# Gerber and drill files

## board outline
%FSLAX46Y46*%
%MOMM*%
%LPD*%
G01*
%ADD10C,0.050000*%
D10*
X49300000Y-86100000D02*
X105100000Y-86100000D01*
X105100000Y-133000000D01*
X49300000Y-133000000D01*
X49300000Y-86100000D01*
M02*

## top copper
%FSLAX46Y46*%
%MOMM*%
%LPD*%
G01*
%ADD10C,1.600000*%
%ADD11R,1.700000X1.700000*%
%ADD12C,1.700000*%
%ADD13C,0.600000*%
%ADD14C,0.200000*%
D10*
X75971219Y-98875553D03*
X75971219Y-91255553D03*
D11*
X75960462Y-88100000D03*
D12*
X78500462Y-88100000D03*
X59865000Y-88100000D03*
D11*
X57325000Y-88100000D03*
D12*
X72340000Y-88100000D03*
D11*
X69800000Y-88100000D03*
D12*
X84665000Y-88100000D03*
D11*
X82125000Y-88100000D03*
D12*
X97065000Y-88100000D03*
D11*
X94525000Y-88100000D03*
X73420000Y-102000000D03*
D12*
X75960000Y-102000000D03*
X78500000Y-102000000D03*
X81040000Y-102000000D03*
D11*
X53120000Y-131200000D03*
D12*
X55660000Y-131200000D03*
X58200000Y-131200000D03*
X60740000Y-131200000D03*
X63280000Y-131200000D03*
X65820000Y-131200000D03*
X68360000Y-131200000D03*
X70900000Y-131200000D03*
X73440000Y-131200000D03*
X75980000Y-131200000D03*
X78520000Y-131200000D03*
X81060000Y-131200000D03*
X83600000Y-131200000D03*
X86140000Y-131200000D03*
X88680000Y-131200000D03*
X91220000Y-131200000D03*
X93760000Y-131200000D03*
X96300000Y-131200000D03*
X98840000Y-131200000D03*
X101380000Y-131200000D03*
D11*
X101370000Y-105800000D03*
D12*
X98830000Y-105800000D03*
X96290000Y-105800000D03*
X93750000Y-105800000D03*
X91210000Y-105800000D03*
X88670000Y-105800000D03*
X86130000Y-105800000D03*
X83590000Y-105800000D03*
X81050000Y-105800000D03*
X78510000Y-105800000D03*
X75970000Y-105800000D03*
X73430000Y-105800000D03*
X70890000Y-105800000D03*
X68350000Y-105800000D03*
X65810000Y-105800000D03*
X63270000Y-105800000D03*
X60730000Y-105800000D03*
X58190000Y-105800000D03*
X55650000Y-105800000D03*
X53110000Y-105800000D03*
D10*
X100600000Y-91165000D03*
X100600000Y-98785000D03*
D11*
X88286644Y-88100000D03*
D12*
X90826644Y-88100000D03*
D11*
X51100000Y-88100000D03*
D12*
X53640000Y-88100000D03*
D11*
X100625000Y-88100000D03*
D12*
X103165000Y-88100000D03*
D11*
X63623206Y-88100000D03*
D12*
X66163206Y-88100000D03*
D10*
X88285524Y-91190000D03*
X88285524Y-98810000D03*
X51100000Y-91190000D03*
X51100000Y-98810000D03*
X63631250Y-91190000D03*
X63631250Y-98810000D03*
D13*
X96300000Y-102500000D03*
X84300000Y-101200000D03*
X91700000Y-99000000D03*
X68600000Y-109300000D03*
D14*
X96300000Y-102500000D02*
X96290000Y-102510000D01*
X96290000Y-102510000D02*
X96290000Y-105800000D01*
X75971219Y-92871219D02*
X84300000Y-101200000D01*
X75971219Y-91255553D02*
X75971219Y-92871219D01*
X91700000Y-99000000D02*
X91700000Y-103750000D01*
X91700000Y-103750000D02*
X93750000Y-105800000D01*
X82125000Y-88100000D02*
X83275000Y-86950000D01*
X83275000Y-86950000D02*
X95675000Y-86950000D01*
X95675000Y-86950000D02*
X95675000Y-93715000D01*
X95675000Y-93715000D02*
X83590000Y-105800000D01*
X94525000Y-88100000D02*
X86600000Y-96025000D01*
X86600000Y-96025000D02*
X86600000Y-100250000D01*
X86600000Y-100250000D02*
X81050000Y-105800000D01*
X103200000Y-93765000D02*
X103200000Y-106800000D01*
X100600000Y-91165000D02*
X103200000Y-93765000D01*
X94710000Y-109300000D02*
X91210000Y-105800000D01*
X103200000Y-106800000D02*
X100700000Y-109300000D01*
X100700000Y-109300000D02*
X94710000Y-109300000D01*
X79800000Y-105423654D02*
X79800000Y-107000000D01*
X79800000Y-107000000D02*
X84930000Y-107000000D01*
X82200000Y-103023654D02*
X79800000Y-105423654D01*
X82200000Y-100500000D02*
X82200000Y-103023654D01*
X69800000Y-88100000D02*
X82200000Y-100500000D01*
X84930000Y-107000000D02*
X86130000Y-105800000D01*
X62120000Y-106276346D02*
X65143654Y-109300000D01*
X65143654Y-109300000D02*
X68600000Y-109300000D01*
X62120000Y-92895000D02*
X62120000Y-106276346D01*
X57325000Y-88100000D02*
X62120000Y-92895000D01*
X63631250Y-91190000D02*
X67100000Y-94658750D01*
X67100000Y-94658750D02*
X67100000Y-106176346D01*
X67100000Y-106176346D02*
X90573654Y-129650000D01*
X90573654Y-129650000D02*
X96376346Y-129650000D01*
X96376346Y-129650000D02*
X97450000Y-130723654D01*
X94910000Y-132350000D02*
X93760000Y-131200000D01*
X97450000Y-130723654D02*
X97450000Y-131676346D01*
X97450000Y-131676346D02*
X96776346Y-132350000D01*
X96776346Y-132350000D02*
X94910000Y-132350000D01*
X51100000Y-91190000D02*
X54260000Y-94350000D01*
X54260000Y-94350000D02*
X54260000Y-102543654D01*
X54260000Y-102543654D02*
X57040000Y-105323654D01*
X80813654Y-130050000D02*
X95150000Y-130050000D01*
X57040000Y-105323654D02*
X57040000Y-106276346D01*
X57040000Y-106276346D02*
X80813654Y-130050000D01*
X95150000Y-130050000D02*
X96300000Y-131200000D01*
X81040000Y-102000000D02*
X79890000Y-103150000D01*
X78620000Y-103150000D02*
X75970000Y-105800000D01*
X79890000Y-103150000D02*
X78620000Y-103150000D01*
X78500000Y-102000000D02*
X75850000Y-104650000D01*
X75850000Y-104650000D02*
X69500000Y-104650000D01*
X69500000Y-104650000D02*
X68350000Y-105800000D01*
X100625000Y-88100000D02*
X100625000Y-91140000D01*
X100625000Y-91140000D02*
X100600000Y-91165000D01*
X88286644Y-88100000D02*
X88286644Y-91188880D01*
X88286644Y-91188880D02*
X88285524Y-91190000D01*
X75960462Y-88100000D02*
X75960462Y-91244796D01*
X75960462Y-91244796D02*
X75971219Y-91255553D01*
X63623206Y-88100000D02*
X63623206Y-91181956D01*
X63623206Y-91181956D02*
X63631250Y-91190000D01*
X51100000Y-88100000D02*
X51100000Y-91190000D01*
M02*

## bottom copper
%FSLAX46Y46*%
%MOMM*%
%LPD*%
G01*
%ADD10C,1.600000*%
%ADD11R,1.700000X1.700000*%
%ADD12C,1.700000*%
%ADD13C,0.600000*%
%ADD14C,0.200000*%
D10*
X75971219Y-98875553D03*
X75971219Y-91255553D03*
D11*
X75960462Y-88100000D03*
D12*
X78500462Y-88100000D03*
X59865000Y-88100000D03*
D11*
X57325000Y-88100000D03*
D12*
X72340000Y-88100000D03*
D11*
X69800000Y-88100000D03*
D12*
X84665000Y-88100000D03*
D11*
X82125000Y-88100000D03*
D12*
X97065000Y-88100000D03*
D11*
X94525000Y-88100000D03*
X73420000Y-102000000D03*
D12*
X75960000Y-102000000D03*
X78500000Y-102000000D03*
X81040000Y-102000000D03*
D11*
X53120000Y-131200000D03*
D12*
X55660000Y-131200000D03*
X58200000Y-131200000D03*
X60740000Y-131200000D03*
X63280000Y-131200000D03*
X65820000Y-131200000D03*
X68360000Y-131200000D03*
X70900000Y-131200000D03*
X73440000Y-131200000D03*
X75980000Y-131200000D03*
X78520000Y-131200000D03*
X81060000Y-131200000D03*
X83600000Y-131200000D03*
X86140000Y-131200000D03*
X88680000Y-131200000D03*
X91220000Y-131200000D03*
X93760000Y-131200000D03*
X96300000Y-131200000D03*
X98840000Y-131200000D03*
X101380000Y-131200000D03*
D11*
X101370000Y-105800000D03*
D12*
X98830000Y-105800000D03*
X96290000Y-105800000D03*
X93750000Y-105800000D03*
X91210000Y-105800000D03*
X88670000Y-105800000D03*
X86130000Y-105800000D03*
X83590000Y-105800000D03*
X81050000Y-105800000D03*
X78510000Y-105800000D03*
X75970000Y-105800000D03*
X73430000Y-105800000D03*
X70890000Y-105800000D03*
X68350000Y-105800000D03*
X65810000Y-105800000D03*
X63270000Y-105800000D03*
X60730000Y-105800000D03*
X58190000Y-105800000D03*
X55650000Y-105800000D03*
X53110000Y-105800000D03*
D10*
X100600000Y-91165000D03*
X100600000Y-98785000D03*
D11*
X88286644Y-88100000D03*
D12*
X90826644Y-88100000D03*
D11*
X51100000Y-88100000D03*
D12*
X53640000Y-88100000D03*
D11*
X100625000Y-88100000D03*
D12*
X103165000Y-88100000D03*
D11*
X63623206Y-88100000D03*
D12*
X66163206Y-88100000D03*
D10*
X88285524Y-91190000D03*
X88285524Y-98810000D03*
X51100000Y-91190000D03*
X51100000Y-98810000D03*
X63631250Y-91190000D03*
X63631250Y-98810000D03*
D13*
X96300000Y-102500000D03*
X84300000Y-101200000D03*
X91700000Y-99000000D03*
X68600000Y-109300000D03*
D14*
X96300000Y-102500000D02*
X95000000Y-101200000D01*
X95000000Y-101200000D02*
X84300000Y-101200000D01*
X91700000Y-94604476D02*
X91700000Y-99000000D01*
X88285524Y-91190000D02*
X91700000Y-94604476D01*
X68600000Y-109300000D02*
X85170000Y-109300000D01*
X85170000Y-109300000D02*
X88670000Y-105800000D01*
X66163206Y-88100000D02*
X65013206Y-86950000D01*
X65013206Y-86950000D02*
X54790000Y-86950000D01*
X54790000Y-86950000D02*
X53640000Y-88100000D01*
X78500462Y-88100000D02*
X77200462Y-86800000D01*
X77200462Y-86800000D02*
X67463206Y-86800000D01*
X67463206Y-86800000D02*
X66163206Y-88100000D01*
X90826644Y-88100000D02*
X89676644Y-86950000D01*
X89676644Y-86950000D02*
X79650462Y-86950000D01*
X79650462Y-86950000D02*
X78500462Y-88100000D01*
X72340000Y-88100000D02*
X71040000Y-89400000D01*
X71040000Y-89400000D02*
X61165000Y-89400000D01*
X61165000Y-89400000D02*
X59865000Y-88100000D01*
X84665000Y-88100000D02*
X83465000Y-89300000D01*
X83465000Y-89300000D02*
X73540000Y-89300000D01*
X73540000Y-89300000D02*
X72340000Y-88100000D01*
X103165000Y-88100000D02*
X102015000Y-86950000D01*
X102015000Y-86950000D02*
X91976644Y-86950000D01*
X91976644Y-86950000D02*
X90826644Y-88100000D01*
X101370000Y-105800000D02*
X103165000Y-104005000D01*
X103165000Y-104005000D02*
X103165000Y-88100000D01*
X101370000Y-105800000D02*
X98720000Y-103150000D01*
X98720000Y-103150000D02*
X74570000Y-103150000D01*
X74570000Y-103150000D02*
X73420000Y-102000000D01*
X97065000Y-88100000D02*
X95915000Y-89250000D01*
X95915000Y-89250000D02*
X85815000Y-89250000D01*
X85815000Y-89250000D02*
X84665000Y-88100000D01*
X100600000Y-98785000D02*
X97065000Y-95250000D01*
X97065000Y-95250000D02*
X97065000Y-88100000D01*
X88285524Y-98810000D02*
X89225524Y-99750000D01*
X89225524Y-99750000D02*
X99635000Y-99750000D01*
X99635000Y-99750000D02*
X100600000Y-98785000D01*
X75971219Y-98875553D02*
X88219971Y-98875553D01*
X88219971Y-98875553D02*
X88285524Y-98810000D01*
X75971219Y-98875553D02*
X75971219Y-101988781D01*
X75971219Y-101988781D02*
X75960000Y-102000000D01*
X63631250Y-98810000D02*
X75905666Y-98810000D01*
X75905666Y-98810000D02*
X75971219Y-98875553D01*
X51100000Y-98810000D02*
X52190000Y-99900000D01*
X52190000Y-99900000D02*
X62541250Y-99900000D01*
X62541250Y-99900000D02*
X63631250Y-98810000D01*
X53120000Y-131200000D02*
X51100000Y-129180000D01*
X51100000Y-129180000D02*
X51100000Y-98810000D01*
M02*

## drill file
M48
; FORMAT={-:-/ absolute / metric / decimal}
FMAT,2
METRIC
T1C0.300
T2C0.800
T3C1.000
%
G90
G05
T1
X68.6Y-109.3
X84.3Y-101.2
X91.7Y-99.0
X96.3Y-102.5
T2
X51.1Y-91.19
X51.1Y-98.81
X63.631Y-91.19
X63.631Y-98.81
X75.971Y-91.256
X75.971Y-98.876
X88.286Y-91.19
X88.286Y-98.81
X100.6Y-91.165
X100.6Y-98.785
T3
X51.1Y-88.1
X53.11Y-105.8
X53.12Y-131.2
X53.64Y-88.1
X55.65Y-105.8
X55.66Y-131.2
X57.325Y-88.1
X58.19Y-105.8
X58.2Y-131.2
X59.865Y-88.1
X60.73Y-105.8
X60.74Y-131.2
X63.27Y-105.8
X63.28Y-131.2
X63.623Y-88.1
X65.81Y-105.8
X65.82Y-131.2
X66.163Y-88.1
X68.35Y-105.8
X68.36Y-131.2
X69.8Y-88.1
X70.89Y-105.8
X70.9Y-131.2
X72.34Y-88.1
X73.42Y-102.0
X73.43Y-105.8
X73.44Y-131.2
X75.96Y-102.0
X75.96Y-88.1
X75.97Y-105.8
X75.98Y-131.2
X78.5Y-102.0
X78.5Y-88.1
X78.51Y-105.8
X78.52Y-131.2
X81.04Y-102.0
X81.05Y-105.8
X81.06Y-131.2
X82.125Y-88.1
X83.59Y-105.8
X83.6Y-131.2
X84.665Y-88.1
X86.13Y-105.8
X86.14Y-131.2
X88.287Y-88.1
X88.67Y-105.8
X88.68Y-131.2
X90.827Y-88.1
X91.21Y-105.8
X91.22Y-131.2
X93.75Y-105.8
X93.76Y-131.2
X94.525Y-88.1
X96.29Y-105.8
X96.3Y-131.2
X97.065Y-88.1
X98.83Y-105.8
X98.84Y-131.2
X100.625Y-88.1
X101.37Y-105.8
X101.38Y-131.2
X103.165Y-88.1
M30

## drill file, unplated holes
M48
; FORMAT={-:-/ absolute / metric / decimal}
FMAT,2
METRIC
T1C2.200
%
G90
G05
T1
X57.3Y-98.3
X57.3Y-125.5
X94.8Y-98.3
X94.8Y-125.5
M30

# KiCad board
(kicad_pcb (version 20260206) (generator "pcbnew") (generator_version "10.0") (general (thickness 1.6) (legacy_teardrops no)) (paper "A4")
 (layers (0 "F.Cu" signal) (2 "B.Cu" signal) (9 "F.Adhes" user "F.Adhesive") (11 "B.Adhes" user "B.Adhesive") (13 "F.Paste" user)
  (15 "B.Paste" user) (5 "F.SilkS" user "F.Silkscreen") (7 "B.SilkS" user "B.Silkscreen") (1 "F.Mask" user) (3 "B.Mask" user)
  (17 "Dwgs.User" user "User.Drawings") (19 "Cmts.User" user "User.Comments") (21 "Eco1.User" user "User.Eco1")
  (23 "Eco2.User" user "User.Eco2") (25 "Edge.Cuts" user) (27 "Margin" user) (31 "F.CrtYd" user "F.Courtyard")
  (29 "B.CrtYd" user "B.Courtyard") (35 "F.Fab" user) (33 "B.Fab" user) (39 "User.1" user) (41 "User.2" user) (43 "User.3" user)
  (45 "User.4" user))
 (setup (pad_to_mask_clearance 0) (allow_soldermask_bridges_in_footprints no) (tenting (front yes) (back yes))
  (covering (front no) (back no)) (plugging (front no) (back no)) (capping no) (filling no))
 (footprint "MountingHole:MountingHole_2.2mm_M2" (layer "F.Cu") (at 94.8 125.5)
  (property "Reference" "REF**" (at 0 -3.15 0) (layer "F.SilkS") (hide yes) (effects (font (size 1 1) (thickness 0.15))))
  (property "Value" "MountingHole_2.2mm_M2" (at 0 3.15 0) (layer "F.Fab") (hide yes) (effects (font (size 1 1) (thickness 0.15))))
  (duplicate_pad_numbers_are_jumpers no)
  (pad "" np_thru_hole circle (at 0 0) (size 2.2 2.2) (drill 2.2) (layers "*.Cu" "*.Mask")))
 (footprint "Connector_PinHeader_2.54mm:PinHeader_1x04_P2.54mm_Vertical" (layer "F.Cu") (at 73.42 102 90)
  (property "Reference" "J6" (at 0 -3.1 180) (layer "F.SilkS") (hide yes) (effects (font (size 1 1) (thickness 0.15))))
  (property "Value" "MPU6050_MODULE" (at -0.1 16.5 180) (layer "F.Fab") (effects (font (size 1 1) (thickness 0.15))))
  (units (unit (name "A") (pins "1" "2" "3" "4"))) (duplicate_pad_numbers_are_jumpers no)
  (pad "1" thru_hole rect (at 0 0 90) (size 1.7 1.7) (drill 1) (layers "*.Cu" "*.Mask") (remove_unused_layers no) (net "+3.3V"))
  (pad "2" thru_hole circle (at 0 2.54 90) (size 1.7 1.7) (drill 1) (layers "*.Cu" "*.Mask") (remove_unused_layers no) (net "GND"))
  (pad "3" thru_hole circle (at 0 5.08 90) (size 1.7 1.7) (drill 1) (layers "*.Cu" "*.Mask") (remove_unused_layers no) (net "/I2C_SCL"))
  (pad "4" thru_hole circle (at 0 7.62 90) (size 1.7 1.7) (drill 1) (layers "*.Cu" "*.Mask") (remove_unused_layers no) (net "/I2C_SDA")))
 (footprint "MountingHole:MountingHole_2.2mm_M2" (layer "F.Cu") (at 94.8 98.3)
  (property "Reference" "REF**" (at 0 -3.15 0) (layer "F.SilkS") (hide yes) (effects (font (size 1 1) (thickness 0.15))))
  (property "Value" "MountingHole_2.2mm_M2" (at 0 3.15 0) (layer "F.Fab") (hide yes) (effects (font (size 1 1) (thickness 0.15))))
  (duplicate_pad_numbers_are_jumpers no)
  (pad "" np_thru_hole circle (at 0 0) (size 2.2 2.2) (drill 2.2) (layers "*.Cu" "*.Mask")))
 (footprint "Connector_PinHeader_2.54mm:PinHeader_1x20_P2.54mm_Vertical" (layer "F.Cu") (at 53.12 131.2 90)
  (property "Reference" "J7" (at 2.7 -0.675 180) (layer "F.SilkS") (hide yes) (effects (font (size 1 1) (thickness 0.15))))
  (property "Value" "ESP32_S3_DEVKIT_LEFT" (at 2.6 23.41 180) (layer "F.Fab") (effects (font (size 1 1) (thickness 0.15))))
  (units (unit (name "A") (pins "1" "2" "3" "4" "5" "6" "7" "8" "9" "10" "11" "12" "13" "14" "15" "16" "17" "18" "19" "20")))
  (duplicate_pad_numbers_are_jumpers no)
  (pad "1" thru_hole rect (at 0 0 90) (size 1.7 1.7) (drill 1) (layers "*.Cu" "*.Mask") (remove_unused_layers no) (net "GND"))
  (pad "2" thru_hole circle (at 0 2.54 90) (size 1.7 1.7) (drill 1) (layers "*.Cu" "*.Mask") (remove_unused_layers no)
   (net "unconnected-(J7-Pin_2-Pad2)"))
  (pad "3" thru_hole circle (at 0 5.08 90) (size 1.7 1.7) (drill 1) (layers "*.Cu" "*.Mask") (remove_unused_layers no)
   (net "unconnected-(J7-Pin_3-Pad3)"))
  (pad "4" thru_hole circle (at 0 7.62 90) (size 1.7 1.7) (drill 1) (layers "*.Cu" "*.Mask") (remove_unused_layers no)
   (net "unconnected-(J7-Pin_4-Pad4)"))
  (pad "5" thru_hole circle (at 0 10.16 90) (size 1.7 1.7) (drill 1) (layers "*.Cu" "*.Mask") (remove_unused_layers no)
   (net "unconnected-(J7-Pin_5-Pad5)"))
  (pad "6" thru_hole circle (at 0 12.7 90) (size 1.7 1.7) (drill 1) (layers "*.Cu" "*.Mask") (remove_unused_layers no)
   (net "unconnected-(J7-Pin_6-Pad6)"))
  (pad "7" thru_hole circle (at 0 15.24 90) (size 1.7 1.7) (drill 1) (layers "*.Cu" "*.Mask") (remove_unused_layers no)
   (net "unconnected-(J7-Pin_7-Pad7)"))
  (pad "8" thru_hole circle (at 0 17.78 90) (size 1.7 1.7) (drill 1) (layers "*.Cu" "*.Mask") (remove_unused_layers no)
   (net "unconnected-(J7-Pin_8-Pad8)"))
  (pad "9" thru_hole circle (at 0 20.32 90) (size 1.7 1.7) (drill 1) (layers "*.Cu" "*.Mask") (remove_unused_layers no)
   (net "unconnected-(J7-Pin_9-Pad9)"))
  (pad "10" thru_hole circle (at 0 22.86 90) (size 1.7 1.7) (drill 1) (layers "*.Cu" "*.Mask") (remove_unused_layers no)
   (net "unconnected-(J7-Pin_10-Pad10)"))
  (pad "11" thru_hole circle (at 0 25.4 90) (size 1.7 1.7) (drill 1) (layers "*.Cu" "*.Mask") (remove_unused_layers no)
   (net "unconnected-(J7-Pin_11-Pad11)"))
  (pad "12" thru_hole circle (at 0 27.94 90) (size 1.7 1.7) (drill 1) (layers "*.Cu" "*.Mask") (remove_unused_layers no)
   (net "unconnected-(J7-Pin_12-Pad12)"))
  (pad "13" thru_hole circle (at 0 30.48 90) (size 1.7 1.7) (drill 1) (layers "*.Cu" "*.Mask") (remove_unused_layers no)
   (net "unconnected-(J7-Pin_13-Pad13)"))
  (pad "14" thru_hole circle (at 0 33.02 90) (size 1.7 1.7) (drill 1) (layers "*.Cu" "*.Mask") (remove_unused_layers no)
   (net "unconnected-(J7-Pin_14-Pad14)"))
  (pad "15" thru_hole circle (at 0 35.56 90) (size 1.7 1.7) (drill 1) (layers "*.Cu" "*.Mask") (remove_unused_layers no)
   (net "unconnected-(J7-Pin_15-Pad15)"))
  (pad "16" thru_hole circle (at 0 38.1 90) (size 1.7 1.7) (drill 1) (layers "*.Cu" "*.Mask") (remove_unused_layers no)
   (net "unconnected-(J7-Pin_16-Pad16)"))
  (pad "17" thru_hole circle (at 0 40.64 90) (size 1.7 1.7) (drill 1) (layers "*.Cu" "*.Mask") (remove_unused_layers no) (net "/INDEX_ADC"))
  (pad "18" thru_hole circle (at 0 43.18 90) (size 1.7 1.7) (drill 1) (layers "*.Cu" "*.Mask") (remove_unused_layers no) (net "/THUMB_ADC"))
  (pad "19" thru_hole circle (at 0 45.72 90) (size 1.7 1.7) (drill 1) (layers "*.Cu" "*.Mask") (remove_unused_layers no)
   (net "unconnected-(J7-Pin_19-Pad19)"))
  (pad "20" thru_hole circle (at 0 48.26 90) (size 1.7 1.7) (drill 1) (layers "*.Cu" "*.Mask") (remove_unused_layers no)
   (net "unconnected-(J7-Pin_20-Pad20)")))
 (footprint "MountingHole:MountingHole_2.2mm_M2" (layer "F.Cu") (at 57.3 98.3)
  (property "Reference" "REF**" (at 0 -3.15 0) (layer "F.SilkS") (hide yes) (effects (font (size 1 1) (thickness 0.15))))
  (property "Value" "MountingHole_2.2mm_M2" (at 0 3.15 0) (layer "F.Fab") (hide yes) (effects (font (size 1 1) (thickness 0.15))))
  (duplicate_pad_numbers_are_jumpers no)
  (pad "" np_thru_hole circle (at 0 0) (size 2.2 2.2) (drill 2.2) (layers "*.Cu" "*.Mask")))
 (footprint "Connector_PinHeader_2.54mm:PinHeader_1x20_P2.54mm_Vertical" (layer "F.Cu") (at 101.37 105.8 -90)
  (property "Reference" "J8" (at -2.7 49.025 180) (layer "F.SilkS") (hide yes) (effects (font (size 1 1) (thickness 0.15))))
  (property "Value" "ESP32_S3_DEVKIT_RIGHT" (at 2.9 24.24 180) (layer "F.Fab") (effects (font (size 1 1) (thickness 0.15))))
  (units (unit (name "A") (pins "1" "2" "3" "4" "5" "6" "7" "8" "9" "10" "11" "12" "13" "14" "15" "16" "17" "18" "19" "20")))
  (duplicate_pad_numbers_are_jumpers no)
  (pad "1" thru_hole rect (at 0 0 270) (size 1.7 1.7) (drill 1) (layers "*.Cu" "*.Mask") (remove_unused_layers no) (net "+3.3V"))
  (pad "2" thru_hole circle (at 0 2.54 270) (size 1.7 1.7) (drill 1) (layers "*.Cu" "*.Mask") (remove_unused_layers no)
   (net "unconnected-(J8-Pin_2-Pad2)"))
  (pad "3" thru_hole circle (at 0 5.08 270) (size 1.7 1.7) (drill 1) (layers "*.Cu" "*.Mask") (remove_unused_layers no) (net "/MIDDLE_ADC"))
  (pad "4" thru_hole circle (at 0 7.62 270) (size 1.7 1.7) (drill 1) (layers "*.Cu" "*.Mask") (remove_unused_layers no) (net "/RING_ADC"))
  (pad "5" thru_hole circle (at 0 10.16 270) (size 1.7 1.7) (drill 1) (layers "*.Cu" "*.Mask") (remove_unused_layers no) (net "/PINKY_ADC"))
  (pad "6" thru_hole circle (at 0 12.7 270) (size 1.7 1.7) (drill 1) (layers "*.Cu" "*.Mask") (remove_unused_layers no) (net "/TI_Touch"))
  (pad "7" thru_hole circle (at 0 15.24 270) (size 1.7 1.7) (drill 1) (layers "*.Cu" "*.Mask") (remove_unused_layers no) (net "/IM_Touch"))
  (pad "8" thru_hole circle (at 0 17.78 270) (size 1.7 1.7) (drill 1) (layers "*.Cu" "*.Mask") (remove_unused_layers no) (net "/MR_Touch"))
  (pad "9" thru_hole circle (at 0 20.32 270) (size 1.7 1.7) (drill 1) (layers "*.Cu" "*.Mask") (remove_unused_layers no) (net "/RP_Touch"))
  (pad "10" thru_hole circle (at 0 22.86 270) (size 1.7 1.7) (drill 1) (layers "*.Cu" "*.Mask") (remove_unused_layers no)
   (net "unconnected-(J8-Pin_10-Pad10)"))
  (pad "11" thru_hole circle (at 0 25.4 270) (size 1.7 1.7) (drill 1) (layers "*.Cu" "*.Mask") (remove_unused_layers no) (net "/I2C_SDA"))
  (pad "12" thru_hole circle (at 0 27.94 270) (size 1.7 1.7) (drill 1) (layers "*.Cu" "*.Mask") (remove_unused_layers no)
   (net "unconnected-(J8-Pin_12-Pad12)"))
  (pad "13" thru_hole circle (at 0 30.48 270) (size 1.7 1.7) (drill 1) (layers "*.Cu" "*.Mask") (remove_unused_layers no)
   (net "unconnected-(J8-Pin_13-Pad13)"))
  (pad "14" thru_hole circle (at 0 33.02 270) (size 1.7 1.7) (drill 1) (layers "*.Cu" "*.Mask") (remove_unused_layers no) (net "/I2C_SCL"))
  (pad "15" thru_hole circle (at 0 35.56 270) (size 1.7 1.7) (drill 1) (layers "*.Cu" "*.Mask") (remove_unused_layers no)
   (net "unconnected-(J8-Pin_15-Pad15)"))
  (pad "16" thru_hole circle (at 0 38.1 270) (size 1.7 1.7) (drill 1) (layers "*.Cu" "*.Mask") (remove_unused_layers no)
   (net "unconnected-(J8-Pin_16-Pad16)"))
  (pad "17" thru_hole circle (at 0 40.64 270) (size 1.7 1.7) (drill 1) (layers "*.Cu" "*.Mask") (remove_unused_layers no)
   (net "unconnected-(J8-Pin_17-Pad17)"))
  (pad "18" thru_hole circle (at 0 43.18 270) (size 1.7 1.7) (drill 1) (layers "*.Cu" "*.Mask") (remove_unused_layers no)
   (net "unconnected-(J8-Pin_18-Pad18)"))
  (pad "19" thru_hole circle (at 0 45.72 270) (size 1.7 1.7) (drill 1) (layers "*.Cu" "*.Mask") (remove_unused_layers no)
   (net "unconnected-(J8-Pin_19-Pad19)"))
  (pad "20" thru_hole circle (at 0 48.26 270) (size 1.7 1.7) (drill 1) (layers "*.Cu" "*.Mask") (remove_unused_layers no)
   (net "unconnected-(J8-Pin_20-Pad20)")))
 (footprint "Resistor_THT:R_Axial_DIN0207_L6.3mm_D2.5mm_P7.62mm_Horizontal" (layer "F.Cu") (at 100.6 91.165 -90)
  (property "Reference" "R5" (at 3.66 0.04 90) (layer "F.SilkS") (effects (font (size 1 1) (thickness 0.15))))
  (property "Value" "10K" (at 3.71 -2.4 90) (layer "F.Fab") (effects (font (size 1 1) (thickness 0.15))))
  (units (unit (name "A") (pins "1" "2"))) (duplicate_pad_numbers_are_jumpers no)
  (pad "1" thru_hole circle (at 0 0 270) (size 1.6 1.6) (drill 0.8) (layers "*.Cu" "*.Mask") (remove_unused_layers no) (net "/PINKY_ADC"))
  (pad "2" thru_hole circle (at 7.62 0 270) (size 1.6 1.6) (drill 0.8) (layers "*.Cu" "*.Mask") (remove_unused_layers no) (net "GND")))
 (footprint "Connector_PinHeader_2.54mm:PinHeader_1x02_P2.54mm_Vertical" (layer "F.Cu") (at 82.125 88.1 90)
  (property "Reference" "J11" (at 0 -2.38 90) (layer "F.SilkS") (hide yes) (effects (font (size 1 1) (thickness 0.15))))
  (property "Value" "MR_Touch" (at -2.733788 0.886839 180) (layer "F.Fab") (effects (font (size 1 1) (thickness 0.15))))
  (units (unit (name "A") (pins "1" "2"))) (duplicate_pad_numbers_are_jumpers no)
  (pad "1" thru_hole rect (at 0 0 90) (size 1.7 1.7) (drill 1) (layers "*.Cu" "*.Mask") (remove_unused_layers no) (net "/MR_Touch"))
  (pad "2" thru_hole circle (at 0 2.54 90) (size 1.7 1.7) (drill 1) (layers "*.Cu" "*.Mask") (remove_unused_layers no) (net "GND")))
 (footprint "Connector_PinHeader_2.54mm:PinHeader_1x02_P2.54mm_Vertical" (layer "F.Cu") (at 94.525 88.1 90)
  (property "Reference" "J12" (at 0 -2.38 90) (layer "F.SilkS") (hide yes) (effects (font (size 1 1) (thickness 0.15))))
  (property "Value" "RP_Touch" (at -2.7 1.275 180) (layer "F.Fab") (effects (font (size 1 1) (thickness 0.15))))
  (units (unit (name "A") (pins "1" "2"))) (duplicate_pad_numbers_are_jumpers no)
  (pad "1" thru_hole rect (at 0 0 90) (size 1.7 1.7) (drill 1) (layers "*.Cu" "*.Mask") (remove_unused_layers no) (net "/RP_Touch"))
  (pad "2" thru_hole circle (at 0 2.54 90) (size 1.7 1.7) (drill 1) (layers "*.Cu" "*.Mask") (remove_unused_layers no) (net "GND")))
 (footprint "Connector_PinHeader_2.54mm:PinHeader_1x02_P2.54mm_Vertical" (layer "F.Cu") (at 88.286644 88.1 90)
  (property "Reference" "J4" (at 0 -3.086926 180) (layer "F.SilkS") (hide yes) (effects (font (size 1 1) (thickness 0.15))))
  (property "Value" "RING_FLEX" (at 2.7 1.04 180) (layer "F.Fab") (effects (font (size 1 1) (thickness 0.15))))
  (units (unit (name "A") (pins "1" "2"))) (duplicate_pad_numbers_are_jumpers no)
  (pad "1" thru_hole rect (at 0 0 90) (size 1.7 1.7) (drill 1) (layers "*.Cu" "*.Mask") (remove_unused_layers no) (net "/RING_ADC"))
  (pad "2" thru_hole circle (at 0 2.54 90) (size 1.7 1.7) (drill 1) (layers "*.Cu" "*.Mask") (remove_unused_layers no) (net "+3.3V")))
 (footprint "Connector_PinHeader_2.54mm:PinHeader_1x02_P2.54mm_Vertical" (layer "F.Cu") (at 51.1 88.1 90)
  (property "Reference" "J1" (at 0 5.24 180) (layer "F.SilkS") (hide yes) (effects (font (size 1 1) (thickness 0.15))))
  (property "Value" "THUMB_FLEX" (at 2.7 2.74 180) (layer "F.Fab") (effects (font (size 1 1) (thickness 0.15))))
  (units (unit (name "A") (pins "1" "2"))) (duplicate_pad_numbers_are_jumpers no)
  (pad "1" thru_hole rect (at 0 0 90) (size 1.7 1.7) (drill 1) (layers "*.Cu" "*.Mask") (remove_unused_layers no) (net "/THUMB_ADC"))
  (pad "2" thru_hole circle (at 0 2.54 90) (size 1.7 1.7) (drill 1) (layers "*.Cu" "*.Mask") (remove_unused_layers no) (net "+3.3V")))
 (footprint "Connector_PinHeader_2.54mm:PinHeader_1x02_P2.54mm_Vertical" (layer "F.Cu") (at 100.625 88.1 90)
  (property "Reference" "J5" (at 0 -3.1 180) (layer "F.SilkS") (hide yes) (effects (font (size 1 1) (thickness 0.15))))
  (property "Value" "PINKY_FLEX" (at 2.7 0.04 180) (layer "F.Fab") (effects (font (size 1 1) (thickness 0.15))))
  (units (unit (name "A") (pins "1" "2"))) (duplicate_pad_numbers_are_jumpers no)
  (pad "1" thru_hole rect (at 0 0 90) (size 1.7 1.7) (drill 1) (layers "*.Cu" "*.Mask") (remove_unused_layers no) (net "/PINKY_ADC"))
  (pad "2" thru_hole circle (at 0 2.54 90) (size 1.7 1.7) (drill 1) (layers "*.Cu" "*.Mask") (remove_unused_layers no) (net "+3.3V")))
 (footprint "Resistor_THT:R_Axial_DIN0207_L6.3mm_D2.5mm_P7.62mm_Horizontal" (layer "F.Cu") (at 75.971219 91.255553 -90)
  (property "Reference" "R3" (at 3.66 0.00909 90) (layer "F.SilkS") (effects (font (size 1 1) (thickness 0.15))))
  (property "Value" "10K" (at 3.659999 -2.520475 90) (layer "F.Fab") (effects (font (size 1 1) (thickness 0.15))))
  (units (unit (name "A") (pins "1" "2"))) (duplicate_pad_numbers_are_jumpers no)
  (pad "1" thru_hole circle (at 0 0 270) (size 1.6 1.6) (drill 0.8) (layers "*.Cu" "*.Mask") (remove_unused_layers no) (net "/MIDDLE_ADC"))
  (pad "2" thru_hole circle (at 7.62 0 270) (size 1.6 1.6) (drill 0.8) (layers "*.Cu" "*.Mask") (remove_unused_layers no) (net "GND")))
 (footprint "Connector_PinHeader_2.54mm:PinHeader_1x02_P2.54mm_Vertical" (layer "F.Cu") (at 63.623206 88.1 90)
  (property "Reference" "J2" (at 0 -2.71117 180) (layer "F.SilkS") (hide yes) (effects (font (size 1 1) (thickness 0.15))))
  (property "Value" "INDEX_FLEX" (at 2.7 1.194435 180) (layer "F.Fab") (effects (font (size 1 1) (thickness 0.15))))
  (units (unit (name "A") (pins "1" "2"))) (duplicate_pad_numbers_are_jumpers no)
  (pad "1" thru_hole rect (at 0 0 90) (size 1.7 1.7) (drill 1) (layers "*.Cu" "*.Mask") (remove_unused_layers no) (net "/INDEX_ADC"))
  (pad "2" thru_hole circle (at 0 2.54 90) (size 1.7 1.7) (drill 1) (layers "*.Cu" "*.Mask") (remove_unused_layers no) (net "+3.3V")))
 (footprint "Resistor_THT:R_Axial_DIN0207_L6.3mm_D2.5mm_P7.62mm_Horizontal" (layer "F.Cu") (at 88.285524 91.19 -90)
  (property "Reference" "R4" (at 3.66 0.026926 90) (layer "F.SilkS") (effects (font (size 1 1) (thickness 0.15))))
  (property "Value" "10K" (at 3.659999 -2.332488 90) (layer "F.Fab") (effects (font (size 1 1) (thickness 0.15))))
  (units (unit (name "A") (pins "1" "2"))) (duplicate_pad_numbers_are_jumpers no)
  (pad "1" thru_hole circle (at 0 0 270) (size 1.6 1.6) (drill 0.8) (layers "*.Cu" "*.Mask") (remove_unused_layers no) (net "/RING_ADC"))
  (pad "2" thru_hole circle (at 7.62 0 270) (size 1.6 1.6) (drill 0.8) (layers "*.Cu" "*.Mask") (remove_unused_layers no) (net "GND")))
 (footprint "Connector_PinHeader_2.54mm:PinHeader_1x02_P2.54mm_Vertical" (layer "F.Cu") (at 57.325 88.1 90)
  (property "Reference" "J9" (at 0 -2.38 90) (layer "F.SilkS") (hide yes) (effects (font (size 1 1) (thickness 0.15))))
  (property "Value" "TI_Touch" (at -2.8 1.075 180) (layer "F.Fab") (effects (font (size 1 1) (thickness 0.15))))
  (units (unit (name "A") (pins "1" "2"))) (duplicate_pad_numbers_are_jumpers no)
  (pad "1" thru_hole rect (at 0 0 90) (size 1.7 1.7) (drill 1) (layers "*.Cu" "*.Mask") (remove_unused_layers no) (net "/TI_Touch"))
  (pad "2" thru_hole circle (at 0 2.54 90) (size 1.7 1.7) (drill 1) (layers "*.Cu" "*.Mask") (remove_unused_layers no) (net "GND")))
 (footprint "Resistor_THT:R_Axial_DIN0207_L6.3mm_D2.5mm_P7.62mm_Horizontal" (layer "F.Cu") (at 51.1 91.19 -90)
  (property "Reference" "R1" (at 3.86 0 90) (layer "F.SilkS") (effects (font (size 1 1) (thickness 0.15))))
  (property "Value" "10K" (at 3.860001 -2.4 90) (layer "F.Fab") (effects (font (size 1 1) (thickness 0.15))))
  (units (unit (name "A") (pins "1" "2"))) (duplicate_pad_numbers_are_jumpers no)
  (pad "1" thru_hole circle (at 0 0 270) (size 1.6 1.6) (drill 0.8) (layers "*.Cu" "*.Mask") (remove_unused_layers no) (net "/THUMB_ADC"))
  (pad "2" thru_hole circle (at 7.62 0 270) (size 1.6 1.6) (drill 0.8) (layers "*.Cu" "*.Mask") (remove_unused_layers no) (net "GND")))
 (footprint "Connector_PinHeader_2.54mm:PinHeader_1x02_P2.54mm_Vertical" (layer "F.Cu") (at 75.960462 88.1 90)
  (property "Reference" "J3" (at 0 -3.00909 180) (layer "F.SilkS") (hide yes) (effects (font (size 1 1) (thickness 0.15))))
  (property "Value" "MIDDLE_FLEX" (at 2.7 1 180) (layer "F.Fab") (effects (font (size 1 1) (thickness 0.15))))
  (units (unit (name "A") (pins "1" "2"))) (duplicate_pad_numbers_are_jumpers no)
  (pad "1" thru_hole rect (at 0 0 90) (size 1.7 1.7) (drill 1) (layers "*.Cu" "*.Mask") (remove_unused_layers no) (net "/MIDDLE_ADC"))
  (pad "2" thru_hole circle (at 0 2.54 90) (size 1.7 1.7) (drill 1) (layers "*.Cu" "*.Mask") (remove_unused_layers no) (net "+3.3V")))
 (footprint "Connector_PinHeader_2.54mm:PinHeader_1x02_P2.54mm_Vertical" (layer "F.Cu") (at 69.8 88.1 90)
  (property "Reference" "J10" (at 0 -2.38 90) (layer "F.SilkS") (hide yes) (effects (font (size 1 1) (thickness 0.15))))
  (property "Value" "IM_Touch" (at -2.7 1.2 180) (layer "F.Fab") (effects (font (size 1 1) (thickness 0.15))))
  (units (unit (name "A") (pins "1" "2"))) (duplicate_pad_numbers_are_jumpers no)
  (pad "1" thru_hole rect (at 0 0 90) (size 1.7 1.7) (drill 1) (layers "*.Cu" "*.Mask") (remove_unused_layers no) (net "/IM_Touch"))
  (pad "2" thru_hole circle (at 0 2.54 90) (size 1.7 1.7) (drill 1) (layers "*.Cu" "*.Mask") (remove_unused_layers no) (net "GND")))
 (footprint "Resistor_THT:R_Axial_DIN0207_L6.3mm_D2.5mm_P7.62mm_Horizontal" (layer "F.Cu") (at 63.63125 91.19 -90)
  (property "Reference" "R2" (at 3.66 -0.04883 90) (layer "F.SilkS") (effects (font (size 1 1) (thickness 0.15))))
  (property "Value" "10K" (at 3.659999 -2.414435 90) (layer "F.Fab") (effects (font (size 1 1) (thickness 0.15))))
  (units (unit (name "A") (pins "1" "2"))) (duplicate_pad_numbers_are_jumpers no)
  (pad "1" thru_hole circle (at 0 0 270) (size 1.6 1.6) (drill 0.8) (layers "*.Cu" "*.Mask") (remove_unused_layers no) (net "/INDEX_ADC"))
  (pad "2" thru_hole circle (at 7.62 0 270) (size 1.6 1.6) (drill 0.8) (layers "*.Cu" "*.Mask") (remove_unused_layers no) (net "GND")))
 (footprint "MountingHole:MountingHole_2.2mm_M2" (layer "F.Cu") (at 57.3 125.5)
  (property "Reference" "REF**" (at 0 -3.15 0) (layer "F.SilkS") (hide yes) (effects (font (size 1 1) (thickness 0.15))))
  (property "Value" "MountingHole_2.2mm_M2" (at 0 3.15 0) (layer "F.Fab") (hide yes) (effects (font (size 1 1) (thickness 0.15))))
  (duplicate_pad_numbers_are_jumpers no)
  (pad "" np_thru_hole circle (at 0 0) (size 2.2 2.2) (drill 2.2) (layers "*.Cu" "*.Mask")))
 (gr_rect (start 49.3 86.1) (end 105.1 133) (stroke (width 0.05) (type default)) (fill no) (layer "Edge.Cuts"))
 (segment (start 77.200462 86.8) (end 67.463206 86.8) (width 0.2) (layer "B.Cu") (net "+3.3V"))
 (segment (start 79.650462 86.95) (end 78.500462 88.1) (width 0.2) (layer "B.Cu") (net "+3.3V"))
 (segment (start 98.72 103.15) (end 74.57 103.15) (width 0.2) (layer "B.Cu") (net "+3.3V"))
 (segment (start 103.165 88.1) (end 102.015 86.95) (width 0.2) (layer "B.Cu") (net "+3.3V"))
 (segment (start 91.976644 86.95) (end 90.826644 88.1) (width 0.2) (layer "B.Cu") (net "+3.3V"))
 (segment (start 90.826644 88.1) (end 89.676644 86.95) (width 0.2) (layer "B.Cu") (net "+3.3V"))
 (segment (start 89.676644 86.95) (end 79.650462 86.95) (width 0.2) (layer "B.Cu") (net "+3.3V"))
 (segment (start 65.013206 86.95) (end 54.79 86.95) (width 0.2) (layer "B.Cu") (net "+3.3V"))
 (segment (start 74.57 103.15) (end 73.42 102) (width 0.2) (layer "B.Cu") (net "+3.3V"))
 (segment (start 103.165 104.005) (end 103.165 88.1) (width 0.2) (layer "B.Cu") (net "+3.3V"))
 (segment (start 102.015 86.95) (end 91.976644 86.95) (width 0.2) (layer "B.Cu") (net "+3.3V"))
 (segment (start 78.500462 88.1) (end 77.200462 86.8) (width 0.2) (layer "B.Cu") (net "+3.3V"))
 (segment (start 67.463206 86.8) (end 66.163206 88.1) (width 0.2) (layer "B.Cu") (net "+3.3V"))
 (segment (start 101.37 105.8) (end 103.165 104.005) (width 0.2) (layer "B.Cu") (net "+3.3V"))
 (segment (start 66.163206 88.1) (end 65.013206 86.95) (width 0.2) (layer "B.Cu") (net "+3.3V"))
 (segment (start 54.79 86.95) (end 53.64 88.1) (width 0.2) (layer "B.Cu") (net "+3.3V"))
 (segment (start 101.37 105.8) (end 98.72 103.15) (width 0.2) (layer "B.Cu") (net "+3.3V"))
 (segment (start 51.1 98.81) (end 52.19 99.9) (width 0.2) (layer "B.Cu") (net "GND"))
 (segment (start 52.19 99.9) (end 62.54125 99.9) (width 0.2) (layer "B.Cu") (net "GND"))
 (segment (start 88.219971 98.875553) (end 88.285524 98.81) (width 0.2) (layer "B.Cu") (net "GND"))
 (segment (start 100.6 98.785) (end 97.065 95.25) (width 0.2) (layer "B.Cu") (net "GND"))
 (segment (start 85.815 89.25) (end 84.665 88.1) (width 0.2) (layer "B.Cu") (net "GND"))
 (segment (start 75.971219 98.875553) (end 88.219971 98.875553) (width 0.2) (layer "B.Cu") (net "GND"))
 (segment (start 63.63125 98.81) (end 75.905666 98.81) (width 0.2) (layer "B.Cu") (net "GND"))
 (segment (start 88.285524 98.81) (end 89.225524 99.75) (width 0.2) (layer "B.Cu") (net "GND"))
 (segment (start 51.1 129.18) (end 51.1 98.81) (width 0.2) (layer "B.Cu") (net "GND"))
 (segment (start 75.971219 101.988781) (end 75.96 102) (width 0.2) (layer "B.Cu") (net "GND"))
 (segment (start 62.54125 99.9) (end 63.63125 98.81) (width 0.2) (layer "B.Cu") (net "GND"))
 (segment (start 53.12 131.2) (end 51.1 129.18) (width 0.2) (layer "B.Cu") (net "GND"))
 (segment (start 89.225524 99.75) (end 99.635 99.75) (width 0.2) (layer "B.Cu") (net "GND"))
 (segment (start 97.065 95.25) (end 97.065 88.1) (width 0.2) (layer "B.Cu") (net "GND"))
 (segment (start 72.34 88.1) (end 71.04 89.4) (width 0.2) (layer "B.Cu") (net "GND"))
 (segment (start 97.065 88.1) (end 95.915 89.25) (width 0.2) (layer "B.Cu") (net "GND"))
 (segment (start 61.165 89.4) (end 59.865 88.1) (width 0.2) (layer "B.Cu") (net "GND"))
 (segment (start 75.971219 98.875553) (end 75.971219 101.988781) (width 0.2) (layer "B.Cu") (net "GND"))
 (segment (start 71.04 89.4) (end 61.165 89.4) (width 0.2) (layer "B.Cu") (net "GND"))
 (segment (start 75.905666 98.81) (end 75.971219 98.875553) (width 0.2) (layer "B.Cu") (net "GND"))
 (segment (start 99.635 99.75) (end 100.6 98.785) (width 0.2) (layer "B.Cu") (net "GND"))
 (segment (start 73.54 89.3) (end 72.34 88.1) (width 0.2) (layer "B.Cu") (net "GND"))
 (segment (start 84.665 88.1) (end 83.465 89.3) (width 0.2) (layer "B.Cu") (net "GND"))
 (segment (start 83.465 89.3) (end 73.54 89.3) (width 0.2) (layer "B.Cu") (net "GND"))
 (segment (start 95.915 89.25) (end 85.815 89.25) (width 0.2) (layer "B.Cu") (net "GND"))
 (segment (start 78.5 102) (end 75.85 104.65) (width 0.2) (layer "F.Cu") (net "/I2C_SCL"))
 (segment (start 69.5 104.65) (end 68.35 105.8) (width 0.2) (layer "F.Cu") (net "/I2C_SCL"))
 (segment (start 75.85 104.65) (end 69.5 104.65) (width 0.2) (layer "F.Cu") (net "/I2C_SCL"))
 (segment (start 78.62 103.15) (end 75.97 105.8) (width 0.2) (layer "F.Cu") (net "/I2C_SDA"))
 (segment (start 81.04 102) (end 79.89 103.15) (width 0.2) (layer "F.Cu") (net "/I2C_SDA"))
 (segment (start 79.89 103.15) (end 78.62 103.15) (width 0.2) (layer "F.Cu") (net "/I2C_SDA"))
 (segment (start 63.623206 91.181956) (end 63.63125 91.19) (width 0.2) (layer "F.Cu") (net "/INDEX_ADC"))
 (segment (start 63.63125 91.19) (end 67.1 94.65875) (width 0.2) (layer "F.Cu") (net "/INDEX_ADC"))
 (segment (start 67.1 106.176346) (end 90.573654 129.65) (width 0.2) (layer "F.Cu") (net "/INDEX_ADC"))
 (segment (start 97.45 130.723654) (end 97.45 131.676346) (width 0.2) (layer "F.Cu") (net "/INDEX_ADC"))
 (segment (start 96.376346 129.65) (end 97.45 130.723654) (width 0.2) (layer "F.Cu") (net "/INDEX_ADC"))
 (segment (start 96.776346 132.35) (end 94.91 132.35) (width 0.2) (layer "F.Cu") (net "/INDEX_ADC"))
 (segment (start 97.45 131.676346) (end 96.776346 132.35) (width 0.2) (layer "F.Cu") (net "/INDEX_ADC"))
 (segment (start 94.91 132.35) (end 93.76 131.2) (width 0.2) (layer "F.Cu") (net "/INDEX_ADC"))
 (segment (start 67.1 94.65875) (end 67.1 106.176346) (width 0.2) (layer "F.Cu") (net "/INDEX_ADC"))
 (segment (start 63.623206 88.1) (end 63.623206 91.181956) (width 0.2) (layer "F.Cu") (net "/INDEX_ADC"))
 (segment (start 90.573654 129.65) (end 96.376346 129.65) (width 0.2) (layer "F.Cu") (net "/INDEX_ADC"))
 (segment (start 51.1 88.1) (end 51.1 91.19) (width 0.2) (layer "F.Cu") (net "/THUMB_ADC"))
 (segment (start 80.813654 130.05) (end 95.15 130.05) (width 0.2) (layer "F.Cu") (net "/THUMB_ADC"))
 (segment (start 57.04 105.323654) (end 57.04 106.276346) (width 0.2) (layer "F.Cu") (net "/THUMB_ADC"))
 (segment (start 51.1 91.19) (end 54.26 94.35) (width 0.2) (layer "F.Cu") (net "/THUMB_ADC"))
 (segment (start 54.26 94.35) (end 54.26 102.543654) (width 0.2) (layer "F.Cu") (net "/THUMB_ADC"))
 (segment (start 57.04 106.276346) (end 80.813654 130.05) (width 0.2) (layer "F.Cu") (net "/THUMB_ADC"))
 (segment (start 54.26 102.543654) (end 57.04 105.323654) (width 0.2) (layer "F.Cu") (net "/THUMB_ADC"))
 (segment (start 95.15 130.05) (end 96.3 131.2) (width 0.2) (layer "F.Cu") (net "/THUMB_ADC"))
 (segment (start 96.29 102.51) (end 96.29 105.8) (width 0.2) (layer "F.Cu") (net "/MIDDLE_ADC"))
 (segment (start 75.971219 91.255553) (end 75.971219 92.871219) (width 0.2) (layer "F.Cu") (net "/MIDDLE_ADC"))
 (segment (start 96.3 102.5) (end 96.29 102.51) (width 0.2) (layer "F.Cu") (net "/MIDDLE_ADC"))
 (segment (start 75.960462 91.244796) (end 75.971219 91.255553) (width 0.2) (layer "F.Cu") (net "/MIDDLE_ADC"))
 (segment (start 75.960462 88.1) (end 75.960462 91.244796) (width 0.2) (layer "F.Cu") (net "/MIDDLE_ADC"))
 (segment (start 75.971219 92.871219) (end 84.3 101.2) (width 0.2) (layer "F.Cu") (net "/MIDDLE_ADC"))
 (via (at 84.3 101.2) (size 0.6) (drill 0.3) (layers "F.Cu" "B.Cu") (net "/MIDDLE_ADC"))
 (via (at 96.3 102.5) (size 0.6) (drill 0.3) (layers "F.Cu" "B.Cu") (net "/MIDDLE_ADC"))
 (segment (start 96.3 102.5) (end 95 101.2) (width 0.2) (layer "B.Cu") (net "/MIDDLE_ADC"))
 (segment (start 95 101.2) (end 84.3 101.2) (width 0.2) (layer "B.Cu") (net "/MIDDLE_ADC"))
 (segment (start 91.7 99) (end 91.7 103.75) (width 0.2) (layer "F.Cu") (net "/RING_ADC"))
 (segment (start 88.286644 91.18888) (end 88.285524 91.19) (width 0.2) (layer "F.Cu") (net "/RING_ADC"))
 (segment (start 88.286644 88.1) (end 88.286644 91.18888) (width 0.2) (layer "F.Cu") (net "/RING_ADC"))
 (segment (start 91.7 103.75) (end 93.75 105.8) (width 0.2) (layer "F.Cu") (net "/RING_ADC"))
 (via (at 91.7 99) (size 0.6) (drill 0.3) (layers "F.Cu" "B.Cu") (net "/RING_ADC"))
 (segment (start 88.285524 91.19) (end 91.7 94.604476) (width 0.2) (layer "B.Cu") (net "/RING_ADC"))
 (segment (start 91.7 94.604476) (end 91.7 99) (width 0.2) (layer "B.Cu") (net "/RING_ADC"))
 (segment (start 100.625 88.1) (end 100.625 91.14) (width 0.2) (layer "F.Cu") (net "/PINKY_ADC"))
 (segment (start 100.7 109.3) (end 94.71 109.3) (width 0.2) (layer "F.Cu") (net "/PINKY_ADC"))
 (segment (start 100.6 91.165) (end 103.2 93.765) (width 0.2) (layer "F.Cu") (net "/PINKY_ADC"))
 (segment (start 100.625 91.14) (end 100.6 91.165) (width 0.2) (layer "F.Cu") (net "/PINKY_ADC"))
 (segment (start 103.2 106.8) (end 100.7 109.3) (width 0.2) (layer "F.Cu") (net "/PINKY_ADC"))
 (segment (start 94.71 109.3) (end 91.21 105.8) (width 0.2) (layer "F.Cu") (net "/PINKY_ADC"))
 (segment (start 103.2 93.765) (end 103.2 106.8) (width 0.2) (layer "F.Cu") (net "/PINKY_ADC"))
 (segment (start 79.8 107) (end 84.93 107) (width 0.2) (layer "F.Cu") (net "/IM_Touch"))
 (segment (start 79.8 105.423654) (end 79.8 107) (width 0.2) (layer "F.Cu") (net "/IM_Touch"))
 (segment (start 69.8 88.1) (end 82.2 100.5) (width 0.2) (layer "F.Cu") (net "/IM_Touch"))
 (segment (start 84.93 107) (end 86.13 105.8) (width 0.2) (layer "F.Cu") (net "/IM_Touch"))
 (segment (start 82.2 100.5) (end 82.2 103.023654) (width 0.2) (layer "F.Cu") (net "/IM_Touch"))
 (segment (start 82.2 103.023654) (end 79.8 105.423654) (width 0.2) (layer "F.Cu") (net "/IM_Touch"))
 (segment (start 95.675 86.95) (end 95.675 93.715) (width 0.2) (layer "F.Cu") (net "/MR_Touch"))
 (segment (start 82.125 88.1) (end 83.275 86.95) (width 0.2) (layer "F.Cu") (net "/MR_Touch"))
 (segment (start 83.275 86.95) (end 95.675 86.95) (width 0.2) (layer "F.Cu") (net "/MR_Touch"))
 (segment (start 95.675 93.715) (end 83.59 105.8) (width 0.2) (layer "F.Cu") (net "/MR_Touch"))
 (segment (start 86.6 100.25) (end 81.05 105.8) (width 0.2) (layer "F.Cu") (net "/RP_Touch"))
 (segment (start 94.525 88.1) (end 86.6 96.025) (width 0.2) (layer "F.Cu") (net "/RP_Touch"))
 (segment (start 86.6 96.025) (end 86.6 100.25) (width 0.2) (layer "F.Cu") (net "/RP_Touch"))
 (segment (start 65.143654 109.3) (end 68.6 109.3) (width 0.2) (layer "F.Cu") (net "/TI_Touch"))
 (segment (start 62.12 92.895) (end 62.12 106.276346) (width 0.2) (layer "F.Cu") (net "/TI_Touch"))
 (segment (start 62.12 106.276346) (end 65.143654 109.3) (width 0.2) (layer "F.Cu") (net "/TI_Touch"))
 (segment (start 57.325 88.1) (end 62.12 92.895) (width 0.2) (layer "F.Cu") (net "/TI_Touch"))
 (via (at 68.6 109.3) (size 0.6) (drill 0.3) (layers "F.Cu" "B.Cu") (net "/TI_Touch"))
 (segment (start 85.17 109.3) (end 88.67 105.8) (width 0.2) (layer "B.Cu") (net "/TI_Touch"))
 (segment (start 68.6 109.3) (end 85.17 109.3) (width 0.2) (layer "B.Cu") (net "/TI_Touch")))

